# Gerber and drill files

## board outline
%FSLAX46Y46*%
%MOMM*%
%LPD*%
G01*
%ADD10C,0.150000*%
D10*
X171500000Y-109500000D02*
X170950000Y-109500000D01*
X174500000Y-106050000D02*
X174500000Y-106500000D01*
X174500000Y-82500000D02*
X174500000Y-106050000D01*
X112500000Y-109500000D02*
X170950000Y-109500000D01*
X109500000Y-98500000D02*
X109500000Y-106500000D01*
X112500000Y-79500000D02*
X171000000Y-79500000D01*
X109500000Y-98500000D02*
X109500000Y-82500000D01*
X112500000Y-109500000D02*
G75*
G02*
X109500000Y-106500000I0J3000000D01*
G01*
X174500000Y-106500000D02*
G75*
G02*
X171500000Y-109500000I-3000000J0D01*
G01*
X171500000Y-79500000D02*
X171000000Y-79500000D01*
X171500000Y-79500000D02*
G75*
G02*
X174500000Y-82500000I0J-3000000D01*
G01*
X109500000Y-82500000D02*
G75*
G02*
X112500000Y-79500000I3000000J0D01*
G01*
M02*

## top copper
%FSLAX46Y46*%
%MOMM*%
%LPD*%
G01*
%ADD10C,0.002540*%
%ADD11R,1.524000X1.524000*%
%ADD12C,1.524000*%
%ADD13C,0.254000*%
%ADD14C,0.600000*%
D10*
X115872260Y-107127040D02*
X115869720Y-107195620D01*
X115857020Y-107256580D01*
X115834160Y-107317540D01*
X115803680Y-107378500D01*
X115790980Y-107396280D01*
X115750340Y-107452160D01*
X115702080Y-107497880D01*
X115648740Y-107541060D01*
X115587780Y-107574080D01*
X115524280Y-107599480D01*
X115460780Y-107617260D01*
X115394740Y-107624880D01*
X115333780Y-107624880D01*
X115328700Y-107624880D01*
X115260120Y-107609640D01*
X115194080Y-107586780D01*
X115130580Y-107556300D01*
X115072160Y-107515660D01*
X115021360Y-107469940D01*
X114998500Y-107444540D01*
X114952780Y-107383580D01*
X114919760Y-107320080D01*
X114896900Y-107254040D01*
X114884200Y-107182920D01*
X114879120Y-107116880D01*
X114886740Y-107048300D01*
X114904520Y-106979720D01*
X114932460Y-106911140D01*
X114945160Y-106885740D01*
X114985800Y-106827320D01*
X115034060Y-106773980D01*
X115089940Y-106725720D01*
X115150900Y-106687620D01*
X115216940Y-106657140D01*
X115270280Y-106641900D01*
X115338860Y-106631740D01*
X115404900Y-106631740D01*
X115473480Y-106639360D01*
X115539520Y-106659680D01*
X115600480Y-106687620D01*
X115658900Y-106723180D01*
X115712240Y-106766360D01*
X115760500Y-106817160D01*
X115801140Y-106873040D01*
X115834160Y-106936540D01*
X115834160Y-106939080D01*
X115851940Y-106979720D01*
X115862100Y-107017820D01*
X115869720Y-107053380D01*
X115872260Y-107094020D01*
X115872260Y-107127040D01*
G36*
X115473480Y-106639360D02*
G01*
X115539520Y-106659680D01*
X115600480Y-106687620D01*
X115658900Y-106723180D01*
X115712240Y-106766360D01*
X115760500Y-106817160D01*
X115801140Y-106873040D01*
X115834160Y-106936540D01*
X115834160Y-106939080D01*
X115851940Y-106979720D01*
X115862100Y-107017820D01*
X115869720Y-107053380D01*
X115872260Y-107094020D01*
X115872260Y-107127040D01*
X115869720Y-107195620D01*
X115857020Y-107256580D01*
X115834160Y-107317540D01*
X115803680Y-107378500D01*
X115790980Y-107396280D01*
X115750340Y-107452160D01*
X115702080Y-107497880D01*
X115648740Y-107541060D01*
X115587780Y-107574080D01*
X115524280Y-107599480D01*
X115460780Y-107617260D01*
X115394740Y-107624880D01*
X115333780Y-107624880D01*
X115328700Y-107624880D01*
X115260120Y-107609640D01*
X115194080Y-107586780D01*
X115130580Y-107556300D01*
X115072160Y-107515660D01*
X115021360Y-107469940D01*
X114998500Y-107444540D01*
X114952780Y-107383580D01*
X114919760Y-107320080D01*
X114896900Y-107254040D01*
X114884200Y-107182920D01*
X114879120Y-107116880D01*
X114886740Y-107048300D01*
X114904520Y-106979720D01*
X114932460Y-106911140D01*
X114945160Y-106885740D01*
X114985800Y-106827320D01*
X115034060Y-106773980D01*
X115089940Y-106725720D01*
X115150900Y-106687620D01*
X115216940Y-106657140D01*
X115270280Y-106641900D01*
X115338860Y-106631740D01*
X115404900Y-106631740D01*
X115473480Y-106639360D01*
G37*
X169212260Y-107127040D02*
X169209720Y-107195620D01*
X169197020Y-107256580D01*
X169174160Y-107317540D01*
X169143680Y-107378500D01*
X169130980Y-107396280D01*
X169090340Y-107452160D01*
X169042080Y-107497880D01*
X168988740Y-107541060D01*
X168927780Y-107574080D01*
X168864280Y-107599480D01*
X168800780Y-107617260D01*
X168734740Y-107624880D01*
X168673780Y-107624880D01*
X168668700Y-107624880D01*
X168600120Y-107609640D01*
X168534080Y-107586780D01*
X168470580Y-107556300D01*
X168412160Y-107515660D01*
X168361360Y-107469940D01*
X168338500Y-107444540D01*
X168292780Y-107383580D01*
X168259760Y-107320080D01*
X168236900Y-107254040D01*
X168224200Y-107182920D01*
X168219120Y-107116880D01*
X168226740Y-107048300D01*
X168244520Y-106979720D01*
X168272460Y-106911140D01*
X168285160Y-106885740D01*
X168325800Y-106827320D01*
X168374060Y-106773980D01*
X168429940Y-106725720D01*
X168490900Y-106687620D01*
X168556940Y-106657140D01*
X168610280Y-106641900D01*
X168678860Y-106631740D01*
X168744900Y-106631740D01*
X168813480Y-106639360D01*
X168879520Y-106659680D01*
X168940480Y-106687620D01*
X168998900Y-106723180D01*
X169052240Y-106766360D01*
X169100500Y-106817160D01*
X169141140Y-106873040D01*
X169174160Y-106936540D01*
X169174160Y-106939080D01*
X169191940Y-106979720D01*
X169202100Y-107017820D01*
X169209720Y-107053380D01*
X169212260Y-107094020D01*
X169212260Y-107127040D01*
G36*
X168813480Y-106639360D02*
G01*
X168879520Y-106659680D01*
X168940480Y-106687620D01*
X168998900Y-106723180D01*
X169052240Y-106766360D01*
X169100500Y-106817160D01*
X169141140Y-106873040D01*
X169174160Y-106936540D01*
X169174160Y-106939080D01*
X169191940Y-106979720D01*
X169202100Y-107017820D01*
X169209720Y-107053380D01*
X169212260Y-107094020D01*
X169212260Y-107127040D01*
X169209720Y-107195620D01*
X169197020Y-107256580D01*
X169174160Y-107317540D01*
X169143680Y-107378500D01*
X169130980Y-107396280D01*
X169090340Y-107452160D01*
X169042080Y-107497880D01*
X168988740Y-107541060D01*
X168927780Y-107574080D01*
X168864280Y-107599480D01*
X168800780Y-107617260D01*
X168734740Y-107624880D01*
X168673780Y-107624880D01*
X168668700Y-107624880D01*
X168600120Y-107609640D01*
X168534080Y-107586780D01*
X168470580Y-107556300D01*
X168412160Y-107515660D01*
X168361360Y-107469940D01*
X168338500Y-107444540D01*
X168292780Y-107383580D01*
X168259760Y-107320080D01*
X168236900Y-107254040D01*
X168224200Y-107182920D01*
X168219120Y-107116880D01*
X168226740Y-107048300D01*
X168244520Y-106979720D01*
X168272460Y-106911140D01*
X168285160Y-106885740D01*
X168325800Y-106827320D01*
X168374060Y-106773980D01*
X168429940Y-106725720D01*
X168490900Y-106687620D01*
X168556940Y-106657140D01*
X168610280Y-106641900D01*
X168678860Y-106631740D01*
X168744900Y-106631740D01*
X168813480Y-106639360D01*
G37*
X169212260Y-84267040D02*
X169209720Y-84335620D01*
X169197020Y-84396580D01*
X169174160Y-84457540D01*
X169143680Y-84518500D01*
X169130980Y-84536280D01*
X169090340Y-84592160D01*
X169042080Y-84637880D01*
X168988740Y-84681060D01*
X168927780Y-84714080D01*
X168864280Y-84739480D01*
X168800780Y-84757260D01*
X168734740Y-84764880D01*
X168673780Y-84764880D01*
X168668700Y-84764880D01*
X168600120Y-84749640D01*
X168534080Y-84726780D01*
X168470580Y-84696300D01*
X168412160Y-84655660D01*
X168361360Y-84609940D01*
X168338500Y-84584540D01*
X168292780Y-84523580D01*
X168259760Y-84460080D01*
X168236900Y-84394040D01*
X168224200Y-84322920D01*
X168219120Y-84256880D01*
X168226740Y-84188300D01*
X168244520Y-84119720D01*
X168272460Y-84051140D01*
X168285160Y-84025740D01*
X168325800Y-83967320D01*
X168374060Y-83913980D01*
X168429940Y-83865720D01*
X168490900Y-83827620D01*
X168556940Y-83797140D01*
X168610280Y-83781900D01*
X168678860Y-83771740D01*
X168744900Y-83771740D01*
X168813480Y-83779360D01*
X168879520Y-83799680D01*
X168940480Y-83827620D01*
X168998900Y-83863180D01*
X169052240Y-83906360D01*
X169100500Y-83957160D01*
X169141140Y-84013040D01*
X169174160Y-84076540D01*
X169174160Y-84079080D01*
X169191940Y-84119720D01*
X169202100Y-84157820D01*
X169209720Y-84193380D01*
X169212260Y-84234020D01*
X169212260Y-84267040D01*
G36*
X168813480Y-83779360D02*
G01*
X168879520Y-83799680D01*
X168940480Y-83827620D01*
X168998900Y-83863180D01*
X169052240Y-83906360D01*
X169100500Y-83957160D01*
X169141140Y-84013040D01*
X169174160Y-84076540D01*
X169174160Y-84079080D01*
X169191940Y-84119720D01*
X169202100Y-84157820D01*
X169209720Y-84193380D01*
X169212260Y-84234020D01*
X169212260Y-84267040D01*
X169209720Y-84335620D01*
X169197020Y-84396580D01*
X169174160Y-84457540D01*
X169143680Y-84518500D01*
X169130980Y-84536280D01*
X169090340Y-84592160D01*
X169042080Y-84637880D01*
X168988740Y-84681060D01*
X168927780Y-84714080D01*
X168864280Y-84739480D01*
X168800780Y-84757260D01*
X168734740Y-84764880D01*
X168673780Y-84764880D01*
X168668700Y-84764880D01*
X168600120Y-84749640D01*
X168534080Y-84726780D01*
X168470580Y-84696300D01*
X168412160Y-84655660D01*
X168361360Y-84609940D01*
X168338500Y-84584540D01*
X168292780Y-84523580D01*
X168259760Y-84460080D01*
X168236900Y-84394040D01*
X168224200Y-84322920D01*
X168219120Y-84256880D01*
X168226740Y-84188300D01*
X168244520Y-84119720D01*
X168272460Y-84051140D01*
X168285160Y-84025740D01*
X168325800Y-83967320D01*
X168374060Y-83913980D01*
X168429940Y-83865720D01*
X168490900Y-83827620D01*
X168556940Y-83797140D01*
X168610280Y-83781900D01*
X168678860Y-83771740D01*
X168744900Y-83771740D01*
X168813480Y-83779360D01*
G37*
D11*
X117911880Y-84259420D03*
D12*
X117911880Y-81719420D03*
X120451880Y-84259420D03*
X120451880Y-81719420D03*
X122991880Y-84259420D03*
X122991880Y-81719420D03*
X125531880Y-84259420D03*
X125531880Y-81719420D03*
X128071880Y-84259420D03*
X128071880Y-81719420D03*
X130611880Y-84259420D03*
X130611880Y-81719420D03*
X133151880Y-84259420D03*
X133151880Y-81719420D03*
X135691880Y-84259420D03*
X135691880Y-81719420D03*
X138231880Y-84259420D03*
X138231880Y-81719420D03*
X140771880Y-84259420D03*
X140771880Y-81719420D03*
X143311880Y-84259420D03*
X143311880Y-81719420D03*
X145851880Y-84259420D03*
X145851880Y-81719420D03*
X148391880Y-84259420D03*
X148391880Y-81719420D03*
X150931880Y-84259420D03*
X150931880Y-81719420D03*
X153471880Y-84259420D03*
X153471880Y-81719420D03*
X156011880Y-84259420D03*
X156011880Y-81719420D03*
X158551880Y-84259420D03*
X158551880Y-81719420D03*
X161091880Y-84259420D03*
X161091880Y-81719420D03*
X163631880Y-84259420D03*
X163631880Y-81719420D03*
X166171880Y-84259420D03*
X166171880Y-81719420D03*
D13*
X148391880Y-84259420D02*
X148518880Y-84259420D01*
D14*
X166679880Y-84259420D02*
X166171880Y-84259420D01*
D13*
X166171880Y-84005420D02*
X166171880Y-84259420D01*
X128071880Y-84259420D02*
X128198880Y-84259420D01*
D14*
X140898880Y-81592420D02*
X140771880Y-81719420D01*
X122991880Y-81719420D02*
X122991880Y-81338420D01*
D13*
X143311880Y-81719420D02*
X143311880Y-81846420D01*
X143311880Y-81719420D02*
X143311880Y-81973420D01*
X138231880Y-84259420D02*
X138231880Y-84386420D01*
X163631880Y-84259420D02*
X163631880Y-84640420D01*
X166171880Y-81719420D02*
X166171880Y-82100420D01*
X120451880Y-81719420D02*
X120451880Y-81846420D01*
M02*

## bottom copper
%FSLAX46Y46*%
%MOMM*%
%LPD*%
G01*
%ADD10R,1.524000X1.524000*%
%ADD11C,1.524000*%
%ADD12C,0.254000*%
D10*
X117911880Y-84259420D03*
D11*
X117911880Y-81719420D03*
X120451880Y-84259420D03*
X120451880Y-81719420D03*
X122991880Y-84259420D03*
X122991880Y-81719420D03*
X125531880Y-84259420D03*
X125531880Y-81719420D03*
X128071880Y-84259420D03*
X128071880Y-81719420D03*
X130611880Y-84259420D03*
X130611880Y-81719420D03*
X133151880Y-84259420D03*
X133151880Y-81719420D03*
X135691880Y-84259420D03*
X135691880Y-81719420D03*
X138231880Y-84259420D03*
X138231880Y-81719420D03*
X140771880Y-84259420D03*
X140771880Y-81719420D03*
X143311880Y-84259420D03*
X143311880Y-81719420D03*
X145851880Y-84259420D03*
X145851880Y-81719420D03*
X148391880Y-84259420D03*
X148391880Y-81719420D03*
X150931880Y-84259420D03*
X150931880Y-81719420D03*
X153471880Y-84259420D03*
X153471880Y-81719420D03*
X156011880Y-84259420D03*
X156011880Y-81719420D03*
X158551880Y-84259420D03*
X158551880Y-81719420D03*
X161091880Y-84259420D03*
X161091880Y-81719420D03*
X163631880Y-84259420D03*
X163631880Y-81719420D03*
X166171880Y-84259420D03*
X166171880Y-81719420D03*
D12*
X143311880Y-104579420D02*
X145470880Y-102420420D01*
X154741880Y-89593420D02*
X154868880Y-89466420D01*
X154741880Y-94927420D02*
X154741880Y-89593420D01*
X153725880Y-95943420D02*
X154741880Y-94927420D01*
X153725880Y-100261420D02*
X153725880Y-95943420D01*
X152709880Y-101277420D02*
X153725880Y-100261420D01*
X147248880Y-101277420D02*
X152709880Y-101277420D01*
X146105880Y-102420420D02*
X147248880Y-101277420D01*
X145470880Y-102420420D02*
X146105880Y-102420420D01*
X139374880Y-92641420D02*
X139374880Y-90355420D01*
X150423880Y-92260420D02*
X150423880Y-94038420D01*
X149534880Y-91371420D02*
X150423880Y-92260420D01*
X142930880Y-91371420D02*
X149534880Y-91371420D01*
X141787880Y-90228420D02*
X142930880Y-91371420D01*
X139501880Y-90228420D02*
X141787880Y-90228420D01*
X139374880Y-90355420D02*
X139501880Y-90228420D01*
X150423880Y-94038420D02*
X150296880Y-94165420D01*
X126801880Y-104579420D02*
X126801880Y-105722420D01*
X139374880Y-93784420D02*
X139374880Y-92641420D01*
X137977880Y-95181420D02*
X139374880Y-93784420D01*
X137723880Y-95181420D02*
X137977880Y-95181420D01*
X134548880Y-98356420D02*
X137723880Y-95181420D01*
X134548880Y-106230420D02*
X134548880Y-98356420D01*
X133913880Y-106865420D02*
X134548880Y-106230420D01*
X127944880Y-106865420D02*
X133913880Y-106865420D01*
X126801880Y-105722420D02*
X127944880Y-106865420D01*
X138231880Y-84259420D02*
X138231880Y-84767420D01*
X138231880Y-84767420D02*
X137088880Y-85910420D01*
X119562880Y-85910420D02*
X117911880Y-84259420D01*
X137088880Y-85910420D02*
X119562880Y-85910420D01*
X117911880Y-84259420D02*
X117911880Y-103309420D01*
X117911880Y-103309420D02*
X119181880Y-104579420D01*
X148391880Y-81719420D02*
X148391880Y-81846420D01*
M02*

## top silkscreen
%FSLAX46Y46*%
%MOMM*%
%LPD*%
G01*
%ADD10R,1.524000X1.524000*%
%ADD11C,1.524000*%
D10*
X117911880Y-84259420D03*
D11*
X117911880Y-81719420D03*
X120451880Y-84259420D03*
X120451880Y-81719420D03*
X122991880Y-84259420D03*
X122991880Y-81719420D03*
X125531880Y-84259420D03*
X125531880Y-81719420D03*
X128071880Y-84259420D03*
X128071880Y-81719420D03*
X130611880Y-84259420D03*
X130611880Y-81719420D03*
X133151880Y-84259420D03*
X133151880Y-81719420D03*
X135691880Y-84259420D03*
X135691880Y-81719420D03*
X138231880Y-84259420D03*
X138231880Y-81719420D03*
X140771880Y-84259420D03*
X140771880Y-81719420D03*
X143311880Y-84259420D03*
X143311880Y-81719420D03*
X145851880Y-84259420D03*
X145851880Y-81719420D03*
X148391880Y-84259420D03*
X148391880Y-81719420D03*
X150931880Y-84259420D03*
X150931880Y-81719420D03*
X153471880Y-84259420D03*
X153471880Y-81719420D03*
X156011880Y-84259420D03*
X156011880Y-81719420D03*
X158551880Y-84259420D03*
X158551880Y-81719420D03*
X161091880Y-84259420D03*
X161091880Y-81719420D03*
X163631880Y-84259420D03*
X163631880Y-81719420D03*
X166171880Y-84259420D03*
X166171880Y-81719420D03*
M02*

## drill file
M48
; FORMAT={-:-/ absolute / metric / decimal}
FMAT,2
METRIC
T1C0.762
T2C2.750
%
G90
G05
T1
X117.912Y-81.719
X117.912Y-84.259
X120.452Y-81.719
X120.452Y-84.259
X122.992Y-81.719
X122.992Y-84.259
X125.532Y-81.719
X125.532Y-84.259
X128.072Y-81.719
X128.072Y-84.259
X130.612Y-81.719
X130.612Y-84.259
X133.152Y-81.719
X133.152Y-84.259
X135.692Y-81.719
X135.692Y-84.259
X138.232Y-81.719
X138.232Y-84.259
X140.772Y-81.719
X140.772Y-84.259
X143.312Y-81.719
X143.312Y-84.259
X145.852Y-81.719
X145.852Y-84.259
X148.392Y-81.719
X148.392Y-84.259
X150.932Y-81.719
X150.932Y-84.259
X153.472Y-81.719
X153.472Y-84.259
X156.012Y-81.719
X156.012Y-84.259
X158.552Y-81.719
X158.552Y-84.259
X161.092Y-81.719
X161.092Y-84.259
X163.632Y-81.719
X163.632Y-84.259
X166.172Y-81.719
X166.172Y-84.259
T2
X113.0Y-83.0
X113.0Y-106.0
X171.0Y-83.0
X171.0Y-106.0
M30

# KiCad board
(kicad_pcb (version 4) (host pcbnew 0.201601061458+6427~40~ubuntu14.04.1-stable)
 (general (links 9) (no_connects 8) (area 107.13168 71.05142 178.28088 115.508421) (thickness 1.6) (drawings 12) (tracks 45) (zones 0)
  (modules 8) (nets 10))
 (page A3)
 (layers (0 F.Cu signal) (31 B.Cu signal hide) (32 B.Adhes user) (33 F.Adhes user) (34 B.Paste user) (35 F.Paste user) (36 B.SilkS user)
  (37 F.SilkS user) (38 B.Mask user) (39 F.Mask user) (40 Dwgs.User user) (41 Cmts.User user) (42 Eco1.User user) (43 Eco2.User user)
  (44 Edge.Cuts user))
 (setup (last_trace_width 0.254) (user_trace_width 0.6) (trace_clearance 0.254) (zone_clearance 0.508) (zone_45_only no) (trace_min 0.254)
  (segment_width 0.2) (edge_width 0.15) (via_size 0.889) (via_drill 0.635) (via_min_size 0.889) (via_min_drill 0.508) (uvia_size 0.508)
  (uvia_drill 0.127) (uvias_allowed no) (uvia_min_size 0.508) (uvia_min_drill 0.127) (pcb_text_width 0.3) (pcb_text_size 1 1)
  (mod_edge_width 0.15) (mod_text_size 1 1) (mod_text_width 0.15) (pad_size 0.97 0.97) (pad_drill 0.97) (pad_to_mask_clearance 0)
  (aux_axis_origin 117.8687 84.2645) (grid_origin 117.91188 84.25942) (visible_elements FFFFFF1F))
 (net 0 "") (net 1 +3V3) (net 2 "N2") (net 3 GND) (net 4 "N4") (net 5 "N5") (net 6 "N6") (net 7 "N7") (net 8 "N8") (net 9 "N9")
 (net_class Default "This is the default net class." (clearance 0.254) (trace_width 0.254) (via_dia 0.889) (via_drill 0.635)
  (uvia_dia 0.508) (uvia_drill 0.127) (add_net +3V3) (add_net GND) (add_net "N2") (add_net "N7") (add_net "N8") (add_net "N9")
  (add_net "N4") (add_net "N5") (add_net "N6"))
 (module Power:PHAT (layer F.Cu) (at 117.91188 82.98942 90)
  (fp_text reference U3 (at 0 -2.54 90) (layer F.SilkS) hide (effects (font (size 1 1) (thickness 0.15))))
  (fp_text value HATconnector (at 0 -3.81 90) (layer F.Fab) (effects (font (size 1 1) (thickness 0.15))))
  (pad 1 thru_hole rect (at -1.27 0 90) (size 1.524 1.524) (drill 0.762) (layers *.Cu *.Mask F.SilkS) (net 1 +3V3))
  (pad 2 thru_hole circle (at 1.27 0 90) (size 1.524 1.524) (drill 0.762) (layers *.Cu *.Mask F.SilkS) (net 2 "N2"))
  (pad 3 thru_hole circle (at -1.27 2.54 90) (size 1.524 1.524) (drill 0.762) (layers *.Cu *.Mask F.SilkS))
  (pad 4 thru_hole circle (at 1.27 2.54 90) (size 1.524 1.524) (drill 0.762) (layers *.Cu *.Mask F.SilkS) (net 2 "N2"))
  (pad 5 thru_hole circle (at -1.27 5.08 90) (size 1.524 1.524) (drill 0.762) (layers *.Cu *.Mask F.SilkS))
  (pad 6 thru_hole circle (at 1.27 5.08 90) (size 1.524 1.524) (drill 0.762) (layers *.Cu *.Mask F.SilkS) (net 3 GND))
  (pad 7 thru_hole circle (at -1.27 7.62 90) (size 1.524 1.524) (drill 0.762) (layers *.Cu *.Mask F.SilkS))
  (pad 8 thru_hole circle (at 1.27 7.62 90) (size 1.524 1.524) (drill 0.762) (layers *.Cu *.Mask F.SilkS))
  (pad 9 thru_hole circle (at -1.27 10.16 90) (size 1.524 1.524) (drill 0.762) (layers *.Cu *.Mask F.SilkS) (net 3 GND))
  (pad 10 thru_hole circle (at 1.27 10.16 90) (size 1.524 1.524) (drill 0.762) (layers *.Cu *.Mask F.SilkS))
  (pad 11 thru_hole circle (at -1.27 12.7 90) (size 1.524 1.524) (drill 0.762) (layers *.Cu *.Mask F.SilkS))
  (pad 12 thru_hole circle (at 1.27 12.7 90) (size 1.524 1.524) (drill 0.762) (layers *.Cu *.Mask F.SilkS))
  (pad 13 thru_hole circle (at -1.27 15.24 90) (size 1.524 1.524) (drill 0.762) (layers *.Cu *.Mask F.SilkS))
  (pad 14 thru_hole circle (at 1.27 15.24 90) (size 1.524 1.524) (drill 0.762) (layers *.Cu *.Mask F.SilkS) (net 3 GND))
  (pad 15 thru_hole circle (at -1.27 17.78 90) (size 1.524 1.524) (drill 0.762) (layers *.Cu *.Mask F.SilkS))
  (pad 16 thru_hole circle (at 1.27 17.78 90) (size 1.524 1.524) (drill 0.762) (layers *.Cu *.Mask F.SilkS))
  (pad 17 thru_hole circle (at -1.27 20.32 90) (size 1.524 1.524) (drill 0.762) (layers *.Cu *.Mask F.SilkS) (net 1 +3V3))
  (pad 18 thru_hole circle (at 1.27 20.32 90) (size 1.524 1.524) (drill 0.762) (layers *.Cu *.Mask F.SilkS))
  (pad 19 thru_hole circle (at -1.27 22.86 90) (size 1.524 1.524) (drill 0.762) (layers *.Cu *.Mask F.SilkS))
  (pad 20 thru_hole circle (at 1.27 22.86 90) (size 1.524 1.524) (drill 0.762) (layers *.Cu *.Mask F.SilkS) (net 3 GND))
  (pad 21 thru_hole circle (at -1.27 25.4 90) (size 1.524 1.524) (drill 0.762) (layers *.Cu *.Mask F.SilkS))
  (pad 22 thru_hole circle (at 1.27 25.4 90) (size 1.524 1.524) (drill 0.762) (layers *.Cu *.Mask F.SilkS) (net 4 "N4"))
  (pad 23 thru_hole circle (at -1.27 27.94 90) (size 1.524 1.524) (drill 0.762) (layers *.Cu *.Mask F.SilkS))
  (pad 24 thru_hole circle (at 1.27 27.94 90) (size 1.524 1.524) (drill 0.762) (layers *.Cu *.Mask F.SilkS))
  (pad 25 thru_hole circle (at -1.27 30.48 90) (size 1.524 1.524) (drill 0.762) (layers *.Cu *.Mask F.SilkS) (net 3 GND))
  (pad 26 thru_hole circle (at 1.27 30.48 90) (size 1.524 1.524) (drill 0.762) (layers *.Cu *.Mask F.SilkS) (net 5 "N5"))
  (pad 27 thru_hole circle (at -1.27 33.02 90) (size 1.524 1.524) (drill 0.762) (layers *.Cu *.Mask F.SilkS))
  (pad 28 thru_hole circle (at 1.27 33.02 90) (size 1.524 1.524) (drill 0.762) (layers *.Cu *.Mask F.SilkS))
  (pad 29 thru_hole circle (at -1.27 35.56 90) (size 1.524 1.524) (drill 0.762) (layers *.Cu *.Mask F.SilkS))
  (pad 30 thru_hole circle (at 1.27 35.56 90) (size 1.524 1.524) (drill 0.762) (layers *.Cu *.Mask F.SilkS) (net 3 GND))
  (pad 31 thru_hole circle (at -1.27 38.1 90) (size 1.524 1.524) (drill 0.762) (layers *.Cu *.Mask F.SilkS))
  (pad 32 thru_hole circle (at 1.27 38.1 90) (size 1.524 1.524) (drill 0.762) (layers *.Cu *.Mask F.SilkS))
  (pad 33 thru_hole circle (at -1.27 40.64 90) (size 1.524 1.524) (drill 0.762) (layers *.Cu *.Mask F.SilkS))
  (pad 34 thru_hole circle (at 1.27 40.64 90) (size 1.524 1.524) (drill 0.762) (layers *.Cu *.Mask F.SilkS) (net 3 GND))
  (pad 35 thru_hole circle (at -1.27 43.18 90) (size 1.524 1.524) (drill 0.762) (layers *.Cu *.Mask F.SilkS) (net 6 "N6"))
  (pad 36 thru_hole circle (at 1.27 43.18 90) (size 1.524 1.524) (drill 0.762) (layers *.Cu *.Mask F.SilkS))
  (pad 37 thru_hole circle (at -1.27 45.72 90) (size 1.524 1.524) (drill 0.762) (layers *.Cu *.Mask F.SilkS) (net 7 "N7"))
  (pad 38 thru_hole circle (at 1.27 45.72 90) (size 1.524 1.524) (drill 0.762) (layers *.Cu *.Mask F.SilkS) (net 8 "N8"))
  (pad 39 thru_hole circle (at -1.27 48.26 90) (size 1.524 1.524) (drill 0.762) (layers *.Cu *.Mask F.SilkS) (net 3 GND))
  (pad 40 thru_hole circle (at 1.27 48.26 90) (size 1.524 1.524) (drill 0.762) (layers *.Cu *.Mask F.SilkS) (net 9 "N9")))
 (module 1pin (layer F.Cu) (at 171 106)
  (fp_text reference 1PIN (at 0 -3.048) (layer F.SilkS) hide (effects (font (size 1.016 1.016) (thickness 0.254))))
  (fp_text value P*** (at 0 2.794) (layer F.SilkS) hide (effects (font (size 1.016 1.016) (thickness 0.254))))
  (pad "" np_thru_hole circle (at 0 0) (size 2.75 2.75) (drill 2.75) (layers *.Cu)))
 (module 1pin (layer F.Cu) (at 113 106)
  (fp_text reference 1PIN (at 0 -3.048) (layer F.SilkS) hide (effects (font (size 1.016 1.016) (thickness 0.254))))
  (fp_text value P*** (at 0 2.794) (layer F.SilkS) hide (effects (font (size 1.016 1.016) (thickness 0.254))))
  (pad "" np_thru_hole circle (at 0 0) (size 2.75 2.75) (drill 2.75) (layers *.Cu)))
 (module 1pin (layer F.Cu) (at 171 83)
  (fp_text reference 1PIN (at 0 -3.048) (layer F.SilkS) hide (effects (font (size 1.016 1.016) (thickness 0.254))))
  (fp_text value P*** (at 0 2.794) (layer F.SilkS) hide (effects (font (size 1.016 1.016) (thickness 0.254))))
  (pad "" np_thru_hole circle (at 0 0) (size 2.75 2.75) (drill 2.75) (layers *.Cu)))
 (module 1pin (layer F.Cu) (at 113 83)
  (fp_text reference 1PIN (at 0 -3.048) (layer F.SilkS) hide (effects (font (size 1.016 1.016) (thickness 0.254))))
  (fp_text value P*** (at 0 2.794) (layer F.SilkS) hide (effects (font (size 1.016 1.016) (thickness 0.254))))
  (pad "" np_thru_hole circle (at 0 0) (size 2.75 2.75) (drill 2.75) (layers *.Cu)))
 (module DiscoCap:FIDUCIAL (layer F.Cu) (at 115.37188 107.11942)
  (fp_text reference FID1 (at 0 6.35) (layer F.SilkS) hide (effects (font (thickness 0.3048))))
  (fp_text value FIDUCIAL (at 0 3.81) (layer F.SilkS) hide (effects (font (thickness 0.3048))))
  (fp_poly
   (pts (xy 0.50038 0.00762) (xy 0.49784 0.0762) (xy 0.48514 0.13716) (xy 0.46228 0.19812) (xy 0.4318 0.25908) (xy 0.4191 0.27686)
    (xy 0.37846 0.33274) (xy 0.3302 0.37846) (xy 0.27686 0.42164) (xy 0.2159 0.45466) (xy 0.1524 0.48006) (xy 0.0889 0.49784)
    (xy 0.02286 0.50546) (xy -0.0381 0.50546) (xy -0.04318 0.50546) (xy -0.11176 0.49022) (xy -0.1778 0.46736) (xy -0.2413 0.43688)
    (xy -0.29972 0.39624) (xy -0.35052 0.35052) (xy -0.37338 0.32512) (xy -0.4191 0.26416) (xy -0.45212 0.20066) (xy -0.47498 0.13462)
    (xy -0.48768 0.0635) (xy -0.49276 -0.00254) (xy -0.48514 -0.07112) (xy -0.46736 -0.1397) (xy -0.43942 -0.20828) (xy -0.42672 -0.23368)
    (xy -0.38608 -0.2921) (xy -0.33782 -0.34544) (xy -0.28194 -0.3937) (xy -0.22098 -0.4318) (xy -0.15494 -0.46228) (xy -0.1016 -0.47752)
    (xy -0.03302 -0.48768) (xy 0.03302 -0.48768) (xy 0.1016 -0.48006) (xy 0.16764 -0.45974) (xy 0.2286 -0.4318) (xy 0.28702 -0.39624)
    (xy 0.34036 -0.35306) (xy 0.38862 -0.30226) (xy 0.42926 -0.24638) (xy 0.46228 -0.18288) (xy 0.46228 -0.18034) (xy 0.48006 -0.1397)
    (xy 0.49022 -0.1016) (xy 0.49784 -0.06604) (xy 0.50038 -0.0254) (xy 0.50038 0.00762) (xy 0.50038 0.00762))
   (layer F.Cu) (width 0.00254)))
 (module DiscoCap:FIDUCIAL (layer F.Cu) (at 168.71188 107.11942)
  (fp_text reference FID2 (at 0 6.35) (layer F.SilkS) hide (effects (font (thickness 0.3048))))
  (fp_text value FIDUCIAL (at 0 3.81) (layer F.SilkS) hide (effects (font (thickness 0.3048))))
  (fp_poly
   (pts (xy 0.50038 0.00762) (xy 0.49784 0.0762) (xy 0.48514 0.13716) (xy 0.46228 0.19812) (xy 0.4318 0.25908) (xy 0.4191 0.27686)
    (xy 0.37846 0.33274) (xy 0.3302 0.37846) (xy 0.27686 0.42164) (xy 0.2159 0.45466) (xy 0.1524 0.48006) (xy 0.0889 0.49784)
    (xy 0.02286 0.50546) (xy -0.0381 0.50546) (xy -0.04318 0.50546) (xy -0.11176 0.49022) (xy -0.1778 0.46736) (xy -0.2413 0.43688)
    (xy -0.29972 0.39624) (xy -0.35052 0.35052) (xy -0.37338 0.32512) (xy -0.4191 0.26416) (xy -0.45212 0.20066) (xy -0.47498 0.13462)
    (xy -0.48768 0.0635) (xy -0.49276 -0.00254) (xy -0.48514 -0.07112) (xy -0.46736 -0.1397) (xy -0.43942 -0.20828) (xy -0.42672 -0.23368)
    (xy -0.38608 -0.2921) (xy -0.33782 -0.34544) (xy -0.28194 -0.3937) (xy -0.22098 -0.4318) (xy -0.15494 -0.46228) (xy -0.1016 -0.47752)
    (xy -0.03302 -0.48768) (xy 0.03302 -0.48768) (xy 0.1016 -0.48006) (xy 0.16764 -0.45974) (xy 0.2286 -0.4318) (xy 0.28702 -0.39624)
    (xy 0.34036 -0.35306) (xy 0.38862 -0.30226) (xy 0.42926 -0.24638) (xy 0.46228 -0.18288) (xy 0.46228 -0.18034) (xy 0.48006 -0.1397)
    (xy 0.49022 -0.1016) (xy 0.49784 -0.06604) (xy 0.50038 -0.0254) (xy 0.50038 0.00762) (xy 0.50038 0.00762))
   (layer F.Cu) (width 0.00254)))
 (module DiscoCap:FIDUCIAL (layer F.Cu) (at 168.71188 84.25942)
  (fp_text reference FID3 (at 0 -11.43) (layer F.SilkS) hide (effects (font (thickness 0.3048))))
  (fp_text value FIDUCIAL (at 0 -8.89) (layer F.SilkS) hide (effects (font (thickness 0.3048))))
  (fp_poly
   (pts (xy 0.50038 0.00762) (xy 0.49784 0.0762) (xy 0.48514 0.13716) (xy 0.46228 0.19812) (xy 0.4318 0.25908) (xy 0.4191 0.27686)
    (xy 0.37846 0.33274) (xy 0.3302 0.37846) (xy 0.27686 0.42164) (xy 0.2159 0.45466) (xy 0.1524 0.48006) (xy 0.0889 0.49784)
    (xy 0.02286 0.50546) (xy -0.0381 0.50546) (xy -0.04318 0.50546) (xy -0.11176 0.49022) (xy -0.1778 0.46736) (xy -0.2413 0.43688)
    (xy -0.29972 0.39624) (xy -0.35052 0.35052) (xy -0.37338 0.32512) (xy -0.4191 0.26416) (xy -0.45212 0.20066) (xy -0.47498 0.13462)
    (xy -0.48768 0.0635) (xy -0.49276 -0.00254) (xy -0.48514 -0.07112) (xy -0.46736 -0.1397) (xy -0.43942 -0.20828) (xy -0.42672 -0.23368)
    (xy -0.38608 -0.2921) (xy -0.33782 -0.34544) (xy -0.28194 -0.3937) (xy -0.22098 -0.4318) (xy -0.15494 -0.46228) (xy -0.1016 -0.47752)
    (xy -0.03302 -0.48768) (xy 0.03302 -0.48768) (xy 0.1016 -0.48006) (xy 0.16764 -0.45974) (xy 0.2286 -0.4318) (xy 0.28702 -0.39624)
    (xy 0.34036 -0.35306) (xy 0.38862 -0.30226) (xy 0.42926 -0.24638) (xy 0.46228 -0.18288) (xy 0.46228 -0.18034) (xy 0.48006 -0.1397)
    (xy 0.49022 -0.1016) (xy 0.49784 -0.06604) (xy 0.50038 -0.0254) (xy 0.50038 0.00762) (xy 0.50038 0.00762))
   (layer F.Cu) (width 0.00254)))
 (gr_line (start 171.5 109.5) (end 170.95 109.5) (angle 90) (layer Edge.Cuts) (width 0.15))
 (gr_line (start 174.5 106.05) (end 174.5 106.5) (angle 90) (layer Edge.Cuts) (width 0.15))
 (gr_line (start 174.5 82.5) (end 174.5 106.05) (angle 90) (layer Edge.Cuts) (width 0.15))
 (gr_line (start 112.5 109.5) (end 170.95 109.5) (angle 90) (layer Edge.Cuts) (width 0.15))
 (gr_line (start 109.5 98.5) (end 109.5 106.5) (angle 90) (layer Edge.Cuts) (width 0.15))
 (gr_line (start 112.5 79.5) (end 171 79.5) (angle 90) (layer Edge.Cuts) (width 0.15))
 (gr_line (start 109.5 98.5) (end 109.5 82.5) (angle 90) (layer Edge.Cuts) (width 0.15))
 (gr_arc (start 112.5 106.5) (end 112.5 109.5) (angle 90) (layer Edge.Cuts) (width 0.15))
 (gr_arc (start 171.5 106.5) (end 174.5 106.5) (angle 90) (layer Edge.Cuts) (width 0.15))
 (gr_line (start 171.5 79.5) (end 171 79.5) (angle 90) (layer Edge.Cuts) (width 0.15))
 (gr_arc (start 171.5 82.5) (end 171.5 79.5) (angle 90) (layer Edge.Cuts) (width 0.15))
 (gr_arc (start 112.5 82.5) (end 109.5 82.5) (angle 90) (layer Edge.Cuts) (width 0.15))
 (segment (start 143.31188 104.57942) (end 145.47088 102.42042) (width 0.254) (layer B.Cu) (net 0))
 (segment (start 154.74188 89.59342) (end 154.86888 89.46642) (width 0.254) (layer B.Cu) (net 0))
 (segment (start 154.74188 94.92742) (end 154.74188 89.59342) (width 0.254) (layer B.Cu) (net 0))
 (segment (start 153.72588 95.94342) (end 154.74188 94.92742) (width 0.254) (layer B.Cu) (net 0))
 (segment (start 153.72588 100.26142) (end 153.72588 95.94342) (width 0.254) (layer B.Cu) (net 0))
 (segment (start 152.70988 101.27742) (end 153.72588 100.26142) (width 0.254) (layer B.Cu) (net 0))
 (segment (start 147.24888 101.27742) (end 152.70988 101.27742) (width 0.254) (layer B.Cu) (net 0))
 (segment (start 146.10588 102.42042) (end 147.24888 101.27742) (width 0.254) (layer B.Cu) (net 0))
 (segment (start 145.47088 102.42042) (end 146.10588 102.42042) (width 0.254) (layer B.Cu) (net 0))
 (segment (start 139.37488 92.64142) (end 139.37488 90.35542) (width 0.254) (layer B.Cu) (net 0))
 (segment (start 150.42388 92.26042) (end 150.42388 94.03842) (width 0.254) (layer B.Cu) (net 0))
 (segment (start 149.53488 91.37142) (end 150.42388 92.26042) (width 0.254) (layer B.Cu) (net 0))
 (segment (start 142.93088 91.37142) (end 149.53488 91.37142) (width 0.254) (layer B.Cu) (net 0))
 (segment (start 141.78788 90.22842) (end 142.93088 91.37142) (width 0.254) (layer B.Cu) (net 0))
 (segment (start 139.50188 90.22842) (end 141.78788 90.22842) (width 0.254) (layer B.Cu) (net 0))
 (segment (start 139.37488 90.35542) (end 139.50188 90.22842) (width 0.254) (layer B.Cu) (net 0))
 (segment (start 150.42388 94.03842) (end 150.29688 94.16542) (width 0.254) (layer B.Cu) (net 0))
 (segment (start 126.80188 104.57942) (end 126.80188 105.72242) (width 0.254) (layer B.Cu) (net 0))
 (segment (start 139.37488 93.78442) (end 139.37488 92.64142) (width 0.254) (layer B.Cu) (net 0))
 (segment (start 137.97788 95.18142) (end 139.37488 93.78442) (width 0.254) (layer B.Cu) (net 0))
 (segment (start 137.72388 95.18142) (end 137.97788 95.18142) (width 0.254) (layer B.Cu) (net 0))
 (segment (start 134.54888 98.35642) (end 137.72388 95.18142) (width 0.254) (layer B.Cu) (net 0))
 (segment (start 134.54888 106.23042) (end 134.54888 98.35642) (width 0.254) (layer B.Cu) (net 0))
 (segment (start 133.91388 106.86542) (end 134.54888 106.23042) (width 0.254) (layer B.Cu) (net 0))
 (segment (start 127.94488 106.86542) (end 133.91388 106.86542) (width 0.254) (layer B.Cu) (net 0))
 (segment (start 126.80188 105.72242) (end 127.94488 106.86542) (width 0.254) (layer B.Cu) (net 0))
 (segment (start 148.39188 84.25942) (end 148.51888 84.25942) (width 0.254) (layer F.Cu) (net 3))
 (segment (start 166.67988 84.25942) (end 166.17188 84.25942) (width 0.6) (layer F.Cu) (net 3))
 (segment (start 166.17188 84.00542) (end 166.17188 84.25942) (width 0.254) (layer F.Cu) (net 3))
 (segment (start 128.07188 84.25942) (end 128.19888 84.25942) (width 0.254) (layer F.Cu) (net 3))
 (segment (start 140.89888 81.59242) (end 140.77188 81.71942) (width 0.6) (layer F.Cu) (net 3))
 (segment (start 122.99188 81.71942) (end 122.99188 81.33842) (width 0.6) (layer F.Cu) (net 3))
 (segment (start 143.31188 81.71942) (end 143.31188 81.84642) (width 0.254) (layer F.Cu) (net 4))
 (segment (start 143.31188 81.71942) (end 143.31188 81.97342) (width 0.254) (layer F.Cu) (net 4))
 (segment (start 138.23188 84.25942) (end 138.23188 84.76742) (width 0.254) (layer B.Cu) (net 1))
 (segment (start 138.23188 84.76742) (end 137.08888 85.91042) (width 0.254) (layer B.Cu) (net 1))
 (segment (start 119.56288 85.91042) (end 117.91188 84.25942) (width 0.254) (layer B.Cu) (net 1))
 (segment (start 137.08888 85.91042) (end 119.56288 85.91042) (width 0.254) (layer B.Cu) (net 1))
 (segment (start 117.91188 84.25942) (end 117.91188 103.30942) (width 0.254) (layer B.Cu) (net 1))
 (segment (start 117.91188 103.30942) (end 119.18188 104.57942) (width 0.254) (layer B.Cu) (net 1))
 (segment (start 138.23188 84.25942) (end 138.23188 84.38642) (width 0.254) (layer F.Cu) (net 1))
 (segment (start 163.63188 84.25942) (end 163.63188 84.64042) (width 0.254) (layer F.Cu) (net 7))
 (segment (start 166.17188 81.71942) (end 166.17188 82.10042) (width 0.254) (layer F.Cu) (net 9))
 (segment (start 148.39188 81.71942) (end 148.39188 81.84642) (width 0.254) (layer B.Cu) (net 5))
 (segment (start 120.45188 81.71942) (end 120.45188 81.84642) (width 0.254) (layer F.Cu) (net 2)))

